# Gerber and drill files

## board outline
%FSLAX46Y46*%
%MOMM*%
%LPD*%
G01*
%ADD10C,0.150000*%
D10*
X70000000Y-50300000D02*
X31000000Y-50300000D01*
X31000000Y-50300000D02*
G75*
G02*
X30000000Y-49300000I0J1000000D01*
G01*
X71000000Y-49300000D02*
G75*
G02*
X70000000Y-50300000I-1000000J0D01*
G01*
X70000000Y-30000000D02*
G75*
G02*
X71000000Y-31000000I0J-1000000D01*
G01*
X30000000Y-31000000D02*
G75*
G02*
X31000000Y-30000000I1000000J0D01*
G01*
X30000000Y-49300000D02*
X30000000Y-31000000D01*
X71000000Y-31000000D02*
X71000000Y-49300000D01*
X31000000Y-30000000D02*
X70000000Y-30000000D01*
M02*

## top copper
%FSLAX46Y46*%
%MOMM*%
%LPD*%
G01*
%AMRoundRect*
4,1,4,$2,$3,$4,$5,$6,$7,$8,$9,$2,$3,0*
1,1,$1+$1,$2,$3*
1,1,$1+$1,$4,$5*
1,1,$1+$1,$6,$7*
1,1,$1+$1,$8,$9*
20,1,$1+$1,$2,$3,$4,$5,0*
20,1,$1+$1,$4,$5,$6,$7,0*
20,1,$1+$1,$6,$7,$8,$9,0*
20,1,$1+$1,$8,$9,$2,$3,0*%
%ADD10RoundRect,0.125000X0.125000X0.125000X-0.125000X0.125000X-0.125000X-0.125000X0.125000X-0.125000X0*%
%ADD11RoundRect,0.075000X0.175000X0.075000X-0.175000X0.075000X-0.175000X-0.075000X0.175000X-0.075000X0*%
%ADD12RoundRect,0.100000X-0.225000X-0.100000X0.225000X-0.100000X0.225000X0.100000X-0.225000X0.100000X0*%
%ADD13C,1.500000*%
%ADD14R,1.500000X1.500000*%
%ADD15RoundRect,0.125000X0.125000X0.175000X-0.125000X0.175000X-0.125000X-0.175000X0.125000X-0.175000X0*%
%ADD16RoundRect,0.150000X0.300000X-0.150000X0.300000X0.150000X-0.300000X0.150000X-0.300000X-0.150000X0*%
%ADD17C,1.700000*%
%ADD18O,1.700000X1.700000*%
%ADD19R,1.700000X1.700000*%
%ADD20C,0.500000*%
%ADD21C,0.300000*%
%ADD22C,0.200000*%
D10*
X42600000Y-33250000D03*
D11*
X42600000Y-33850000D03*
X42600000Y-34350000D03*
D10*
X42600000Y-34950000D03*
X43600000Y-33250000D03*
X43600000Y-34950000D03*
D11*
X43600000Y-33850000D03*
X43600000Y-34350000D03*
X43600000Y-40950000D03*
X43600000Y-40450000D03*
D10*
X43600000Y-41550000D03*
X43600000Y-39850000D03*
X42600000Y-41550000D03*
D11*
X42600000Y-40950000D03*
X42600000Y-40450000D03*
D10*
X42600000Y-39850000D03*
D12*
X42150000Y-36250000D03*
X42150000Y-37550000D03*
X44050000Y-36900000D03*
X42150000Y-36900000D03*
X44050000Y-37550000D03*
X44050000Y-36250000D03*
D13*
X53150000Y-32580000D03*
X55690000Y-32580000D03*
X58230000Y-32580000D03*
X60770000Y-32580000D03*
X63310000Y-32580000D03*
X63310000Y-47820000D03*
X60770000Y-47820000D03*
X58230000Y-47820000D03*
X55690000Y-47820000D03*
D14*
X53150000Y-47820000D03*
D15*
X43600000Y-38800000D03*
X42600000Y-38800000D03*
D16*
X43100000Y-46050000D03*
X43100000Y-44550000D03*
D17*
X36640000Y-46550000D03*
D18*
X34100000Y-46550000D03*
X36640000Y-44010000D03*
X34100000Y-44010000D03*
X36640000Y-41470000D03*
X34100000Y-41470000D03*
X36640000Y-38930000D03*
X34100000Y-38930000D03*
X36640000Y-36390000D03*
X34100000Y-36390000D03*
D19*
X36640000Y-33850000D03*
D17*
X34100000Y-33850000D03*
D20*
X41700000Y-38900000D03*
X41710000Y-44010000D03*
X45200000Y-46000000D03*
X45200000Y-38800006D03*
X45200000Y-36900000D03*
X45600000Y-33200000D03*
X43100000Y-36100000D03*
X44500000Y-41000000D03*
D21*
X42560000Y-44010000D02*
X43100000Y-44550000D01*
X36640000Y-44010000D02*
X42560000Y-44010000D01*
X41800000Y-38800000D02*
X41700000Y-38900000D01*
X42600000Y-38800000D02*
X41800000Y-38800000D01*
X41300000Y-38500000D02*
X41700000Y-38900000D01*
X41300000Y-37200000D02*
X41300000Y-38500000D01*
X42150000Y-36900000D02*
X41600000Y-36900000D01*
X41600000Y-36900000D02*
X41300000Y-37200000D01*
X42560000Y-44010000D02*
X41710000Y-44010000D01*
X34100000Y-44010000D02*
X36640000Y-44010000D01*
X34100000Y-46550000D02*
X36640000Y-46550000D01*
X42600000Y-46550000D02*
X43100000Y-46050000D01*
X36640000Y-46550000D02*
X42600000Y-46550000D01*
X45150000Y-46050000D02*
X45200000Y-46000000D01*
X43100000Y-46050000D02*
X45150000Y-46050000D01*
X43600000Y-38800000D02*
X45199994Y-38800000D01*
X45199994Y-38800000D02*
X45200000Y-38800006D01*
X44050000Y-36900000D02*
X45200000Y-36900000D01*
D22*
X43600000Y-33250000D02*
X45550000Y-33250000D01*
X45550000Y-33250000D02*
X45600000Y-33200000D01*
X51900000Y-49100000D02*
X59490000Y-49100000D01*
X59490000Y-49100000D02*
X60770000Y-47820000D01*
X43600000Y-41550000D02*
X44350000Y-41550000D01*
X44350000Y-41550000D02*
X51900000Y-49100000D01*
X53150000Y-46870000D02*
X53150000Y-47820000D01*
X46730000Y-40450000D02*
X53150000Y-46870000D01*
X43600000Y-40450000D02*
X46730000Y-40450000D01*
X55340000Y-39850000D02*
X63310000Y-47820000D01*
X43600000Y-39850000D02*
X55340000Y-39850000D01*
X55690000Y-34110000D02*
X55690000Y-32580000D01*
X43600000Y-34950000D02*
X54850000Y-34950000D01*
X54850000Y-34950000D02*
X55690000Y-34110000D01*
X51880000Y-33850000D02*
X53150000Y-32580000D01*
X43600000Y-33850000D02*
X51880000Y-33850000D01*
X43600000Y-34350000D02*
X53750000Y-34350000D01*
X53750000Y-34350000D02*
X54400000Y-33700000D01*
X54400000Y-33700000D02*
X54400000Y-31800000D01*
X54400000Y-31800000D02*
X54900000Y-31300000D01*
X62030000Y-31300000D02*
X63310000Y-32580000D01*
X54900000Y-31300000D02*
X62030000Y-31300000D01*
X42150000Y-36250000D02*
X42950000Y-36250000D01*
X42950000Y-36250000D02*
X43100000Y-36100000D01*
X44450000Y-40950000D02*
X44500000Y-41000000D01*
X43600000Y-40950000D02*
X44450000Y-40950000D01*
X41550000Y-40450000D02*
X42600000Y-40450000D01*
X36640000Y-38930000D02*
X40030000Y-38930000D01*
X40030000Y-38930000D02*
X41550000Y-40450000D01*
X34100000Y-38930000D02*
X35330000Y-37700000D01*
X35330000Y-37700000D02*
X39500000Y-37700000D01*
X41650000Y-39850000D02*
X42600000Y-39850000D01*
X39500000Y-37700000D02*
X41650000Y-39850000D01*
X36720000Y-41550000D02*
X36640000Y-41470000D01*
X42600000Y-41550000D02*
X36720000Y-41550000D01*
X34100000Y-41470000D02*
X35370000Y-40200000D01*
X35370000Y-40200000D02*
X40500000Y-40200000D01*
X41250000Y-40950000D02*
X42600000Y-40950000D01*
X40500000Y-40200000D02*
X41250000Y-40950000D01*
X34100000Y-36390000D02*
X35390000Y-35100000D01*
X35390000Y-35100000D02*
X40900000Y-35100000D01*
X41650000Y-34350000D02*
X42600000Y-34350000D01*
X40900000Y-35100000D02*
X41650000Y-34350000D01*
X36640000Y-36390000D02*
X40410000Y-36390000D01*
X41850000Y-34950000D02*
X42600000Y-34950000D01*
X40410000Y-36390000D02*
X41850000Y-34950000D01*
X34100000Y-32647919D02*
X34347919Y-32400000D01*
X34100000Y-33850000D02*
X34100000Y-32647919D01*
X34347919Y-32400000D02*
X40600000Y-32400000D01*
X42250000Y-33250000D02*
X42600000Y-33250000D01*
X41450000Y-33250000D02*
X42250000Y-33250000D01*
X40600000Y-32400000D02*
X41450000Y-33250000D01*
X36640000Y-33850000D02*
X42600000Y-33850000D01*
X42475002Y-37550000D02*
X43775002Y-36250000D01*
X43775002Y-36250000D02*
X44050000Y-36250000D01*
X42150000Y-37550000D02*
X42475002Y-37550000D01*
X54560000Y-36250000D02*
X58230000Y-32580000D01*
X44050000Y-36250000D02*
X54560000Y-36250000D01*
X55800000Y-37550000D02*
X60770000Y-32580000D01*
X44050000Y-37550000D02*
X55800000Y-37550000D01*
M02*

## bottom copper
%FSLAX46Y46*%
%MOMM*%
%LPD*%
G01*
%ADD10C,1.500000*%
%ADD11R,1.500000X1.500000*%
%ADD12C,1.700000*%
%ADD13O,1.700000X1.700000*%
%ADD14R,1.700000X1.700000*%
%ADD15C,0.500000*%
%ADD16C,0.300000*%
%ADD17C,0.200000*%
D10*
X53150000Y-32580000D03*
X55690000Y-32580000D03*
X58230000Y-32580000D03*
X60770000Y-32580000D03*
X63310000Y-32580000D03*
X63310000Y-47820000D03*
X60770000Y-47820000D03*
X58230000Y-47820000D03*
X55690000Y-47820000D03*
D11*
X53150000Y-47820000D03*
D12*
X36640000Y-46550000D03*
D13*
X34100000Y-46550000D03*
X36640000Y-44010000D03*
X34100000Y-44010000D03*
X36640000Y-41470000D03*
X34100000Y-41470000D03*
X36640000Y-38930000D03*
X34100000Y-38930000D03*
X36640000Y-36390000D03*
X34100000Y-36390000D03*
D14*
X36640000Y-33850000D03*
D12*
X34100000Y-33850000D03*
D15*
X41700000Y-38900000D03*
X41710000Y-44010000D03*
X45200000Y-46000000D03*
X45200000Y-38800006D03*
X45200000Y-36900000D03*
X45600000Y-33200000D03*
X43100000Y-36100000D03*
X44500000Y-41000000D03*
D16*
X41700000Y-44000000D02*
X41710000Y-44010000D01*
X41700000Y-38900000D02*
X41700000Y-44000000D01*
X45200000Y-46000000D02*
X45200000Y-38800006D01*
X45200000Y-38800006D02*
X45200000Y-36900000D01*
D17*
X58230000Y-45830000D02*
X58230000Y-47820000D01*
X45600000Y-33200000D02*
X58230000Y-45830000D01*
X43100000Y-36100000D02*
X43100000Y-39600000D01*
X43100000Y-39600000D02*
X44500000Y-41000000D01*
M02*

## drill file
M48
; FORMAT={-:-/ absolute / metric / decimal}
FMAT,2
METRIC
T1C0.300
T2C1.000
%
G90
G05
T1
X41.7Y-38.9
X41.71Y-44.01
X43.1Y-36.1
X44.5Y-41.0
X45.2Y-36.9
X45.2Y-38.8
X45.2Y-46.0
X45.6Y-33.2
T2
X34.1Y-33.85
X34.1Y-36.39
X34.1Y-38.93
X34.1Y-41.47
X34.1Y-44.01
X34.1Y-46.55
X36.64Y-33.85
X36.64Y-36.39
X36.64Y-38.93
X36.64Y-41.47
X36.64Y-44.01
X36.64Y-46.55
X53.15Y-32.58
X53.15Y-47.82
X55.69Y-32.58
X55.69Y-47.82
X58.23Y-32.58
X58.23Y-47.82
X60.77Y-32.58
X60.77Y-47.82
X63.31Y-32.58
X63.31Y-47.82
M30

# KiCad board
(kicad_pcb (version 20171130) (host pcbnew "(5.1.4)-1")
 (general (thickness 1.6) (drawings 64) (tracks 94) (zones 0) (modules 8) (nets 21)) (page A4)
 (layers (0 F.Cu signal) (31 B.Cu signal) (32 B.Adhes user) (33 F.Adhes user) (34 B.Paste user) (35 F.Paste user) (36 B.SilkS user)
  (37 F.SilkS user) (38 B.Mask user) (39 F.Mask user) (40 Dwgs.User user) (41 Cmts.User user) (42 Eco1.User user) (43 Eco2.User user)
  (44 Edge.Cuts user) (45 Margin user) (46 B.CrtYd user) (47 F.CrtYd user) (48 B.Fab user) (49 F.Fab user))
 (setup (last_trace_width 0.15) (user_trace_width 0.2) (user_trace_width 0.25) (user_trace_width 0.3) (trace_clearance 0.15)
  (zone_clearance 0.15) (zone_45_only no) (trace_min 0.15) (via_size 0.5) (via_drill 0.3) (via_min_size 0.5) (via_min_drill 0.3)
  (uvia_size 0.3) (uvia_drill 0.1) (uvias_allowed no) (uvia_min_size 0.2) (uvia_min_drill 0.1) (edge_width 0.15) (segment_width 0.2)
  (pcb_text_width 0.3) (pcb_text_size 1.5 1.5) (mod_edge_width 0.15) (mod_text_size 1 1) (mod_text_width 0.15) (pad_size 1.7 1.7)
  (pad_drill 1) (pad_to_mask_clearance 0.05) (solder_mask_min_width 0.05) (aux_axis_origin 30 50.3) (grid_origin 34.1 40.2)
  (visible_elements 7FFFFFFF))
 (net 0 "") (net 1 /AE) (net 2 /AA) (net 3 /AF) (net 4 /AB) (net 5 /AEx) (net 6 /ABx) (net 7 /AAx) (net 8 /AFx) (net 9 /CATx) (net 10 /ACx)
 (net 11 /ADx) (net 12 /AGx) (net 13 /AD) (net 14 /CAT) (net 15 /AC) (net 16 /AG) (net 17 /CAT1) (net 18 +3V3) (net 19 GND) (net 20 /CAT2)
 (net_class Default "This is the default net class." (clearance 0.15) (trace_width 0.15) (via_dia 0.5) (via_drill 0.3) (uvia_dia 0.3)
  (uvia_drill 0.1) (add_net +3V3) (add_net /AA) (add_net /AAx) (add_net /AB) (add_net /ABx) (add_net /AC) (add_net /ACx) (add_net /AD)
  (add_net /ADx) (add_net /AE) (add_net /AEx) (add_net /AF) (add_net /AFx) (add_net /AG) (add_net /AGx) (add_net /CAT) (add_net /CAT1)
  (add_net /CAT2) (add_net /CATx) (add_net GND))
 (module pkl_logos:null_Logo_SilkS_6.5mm (layer B.Cu) (at 52.7 40.2 90)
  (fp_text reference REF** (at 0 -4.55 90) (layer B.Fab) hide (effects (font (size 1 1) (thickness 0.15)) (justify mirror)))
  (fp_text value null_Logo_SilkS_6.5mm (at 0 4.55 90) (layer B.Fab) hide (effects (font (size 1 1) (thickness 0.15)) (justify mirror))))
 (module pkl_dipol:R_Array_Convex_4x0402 (layer F.Cu) (at 43.1 34.1 180) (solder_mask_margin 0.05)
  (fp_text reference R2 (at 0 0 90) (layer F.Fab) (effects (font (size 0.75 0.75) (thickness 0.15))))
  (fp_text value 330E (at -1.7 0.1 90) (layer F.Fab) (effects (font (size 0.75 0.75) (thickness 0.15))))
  (pad 8 smd roundrect (at 0.5 0.85 180) (size 0.5 0.5) (layers F.Cu F.Paste F.Mask) (roundrect_rratio 0.25) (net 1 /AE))
  (pad 6 smd roundrect (at 0.5 0.25 180) (size 0.5 0.3) (layers F.Cu F.Paste F.Mask) (roundrect_rratio 0.25) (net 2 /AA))
  (pad 4 smd roundrect (at 0.5 -0.25 180) (size 0.5 0.3) (layers F.Cu F.Paste F.Mask) (roundrect_rratio 0.25) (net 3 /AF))
  (pad 2 smd roundrect (at 0.5 -0.85 180) (size 0.5 0.5) (layers F.Cu F.Paste F.Mask) (roundrect_rratio 0.25) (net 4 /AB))
  (pad 7 smd roundrect (at -0.5 0.85 180) (size 0.5 0.5) (layers F.Cu F.Paste F.Mask) (roundrect_rratio 0.25) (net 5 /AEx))
  (pad 1 smd roundrect (at -0.5 -0.85 180) (size 0.5 0.5) (layers F.Cu F.Paste F.Mask) (roundrect_rratio 0.25) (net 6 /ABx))
  (pad 5 smd roundrect (at -0.5 0.25 180) (size 0.5 0.3) (layers F.Cu F.Paste F.Mask) (roundrect_rratio 0.25) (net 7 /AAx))
  (pad 3 smd roundrect (at -0.5 -0.25 180) (size 0.5 0.3) (layers F.Cu F.Paste F.Mask) (roundrect_rratio 0.25) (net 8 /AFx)))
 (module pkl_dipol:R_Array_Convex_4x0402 (layer F.Cu) (at 43.1 40.7 180) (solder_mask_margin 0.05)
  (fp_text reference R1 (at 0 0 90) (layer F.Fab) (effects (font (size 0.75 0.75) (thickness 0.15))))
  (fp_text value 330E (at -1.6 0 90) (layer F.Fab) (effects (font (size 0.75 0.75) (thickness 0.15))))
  (pad 3 smd roundrect (at -0.5 -0.25 180) (size 0.5 0.3) (layers F.Cu F.Paste F.Mask) (roundrect_rratio 0.25) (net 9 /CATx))
  (pad 5 smd roundrect (at -0.5 0.25 180) (size 0.5 0.3) (layers F.Cu F.Paste F.Mask) (roundrect_rratio 0.25) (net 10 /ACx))
  (pad 1 smd roundrect (at -0.5 -0.85 180) (size 0.5 0.5) (layers F.Cu F.Paste F.Mask) (roundrect_rratio 0.25) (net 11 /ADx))
  (pad 7 smd roundrect (at -0.5 0.85 180) (size 0.5 0.5) (layers F.Cu F.Paste F.Mask) (roundrect_rratio 0.25) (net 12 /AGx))
  (pad 2 smd roundrect (at 0.5 -0.85 180) (size 0.5 0.5) (layers F.Cu F.Paste F.Mask) (roundrect_rratio 0.25) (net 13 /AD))
  (pad 4 smd roundrect (at 0.5 -0.25 180) (size 0.5 0.3) (layers F.Cu F.Paste F.Mask) (roundrect_rratio 0.25) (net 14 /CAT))
  (pad 6 smd roundrect (at 0.5 0.25 180) (size 0.5 0.3) (layers F.Cu F.Paste F.Mask) (roundrect_rratio 0.25) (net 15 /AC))
  (pad 8 smd roundrect (at 0.5 0.85 180) (size 0.5 0.5) (layers F.Cu F.Paste F.Mask) (roundrect_rratio 0.25) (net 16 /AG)))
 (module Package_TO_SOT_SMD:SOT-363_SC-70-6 (layer F.Cu) (at 43.1 36.9)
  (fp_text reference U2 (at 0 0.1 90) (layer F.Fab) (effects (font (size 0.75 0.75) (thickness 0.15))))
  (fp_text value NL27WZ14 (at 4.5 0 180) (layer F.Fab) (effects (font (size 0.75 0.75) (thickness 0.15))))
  (pad 1 smd roundrect (at -0.95 -0.65) (size 0.65 0.4) (layers F.Cu F.Paste F.Mask) (roundrect_rratio 0.25) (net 9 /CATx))
  (pad 3 smd roundrect (at -0.95 0.65) (size 0.65 0.4) (layers F.Cu F.Paste F.Mask) (roundrect_rratio 0.25) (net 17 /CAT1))
  (pad 5 smd roundrect (at 0.95 0) (size 0.65 0.4) (layers F.Cu F.Paste F.Mask) (roundrect_rratio 0.25) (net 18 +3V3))
  (pad 2 smd roundrect (at -0.95 0) (size 0.65 0.4) (layers F.Cu F.Paste F.Mask) (roundrect_rratio 0.25) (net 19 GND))
  (pad 4 smd roundrect (at 0.95 0.65) (size 0.65 0.4) (layers F.Cu F.Paste F.Mask) (roundrect_rratio 0.25) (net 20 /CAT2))
  (pad 6 smd roundrect (at 0.95 -0.65) (size 0.65 0.4) (layers F.Cu F.Paste F.Mask) (roundrect_rratio 0.25) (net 17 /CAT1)))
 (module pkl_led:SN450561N (layer F.Cu) (at 53.15 47.82 90)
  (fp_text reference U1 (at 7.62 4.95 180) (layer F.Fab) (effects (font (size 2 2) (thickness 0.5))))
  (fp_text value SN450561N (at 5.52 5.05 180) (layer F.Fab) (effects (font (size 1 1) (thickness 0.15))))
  (pad 10 thru_hole circle (at 15.24 0 90) (size 1.5 1.5) (drill 1) (layers *.Cu *.Mask) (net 7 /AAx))
  (pad 9 thru_hole circle (at 15.24 2.54 90) (size 1.5 1.5) (drill 1) (layers *.Cu *.Mask) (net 6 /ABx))
  (pad 8 thru_hole circle (at 15.24 5.08 90) (size 1.5 1.5) (drill 1) (layers *.Cu *.Mask) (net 17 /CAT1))
  (pad 7 thru_hole circle (at 15.24 7.62 90) (size 1.5 1.5) (drill 1) (layers *.Cu *.Mask) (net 20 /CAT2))
  (pad 6 thru_hole circle (at 15.24 10.16 90) (size 1.5 1.5) (drill 1) (layers *.Cu *.Mask) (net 8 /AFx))
  (pad 5 thru_hole circle (at 0 10.16 90) (size 1.5 1.5) (drill 1) (layers *.Cu *.Mask) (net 12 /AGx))
  (pad 4 thru_hole circle (at 0 7.62 90) (size 1.5 1.5) (drill 1) (layers *.Cu *.Mask) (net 11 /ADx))
  (pad 3 thru_hole circle (at 0 5.08 90) (size 1.5 1.5) (drill 1) (layers *.Cu *.Mask) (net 5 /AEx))
  (pad 2 thru_hole circle (at 0 2.54 90) (size 1.5 1.5) (drill 1) (layers *.Cu *.Mask))
  (pad 1 thru_hole rect (at 0 0 90) (size 1.5 1.5) (drill 1) (layers *.Cu *.Mask) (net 10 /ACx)))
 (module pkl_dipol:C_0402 (layer F.Cu) (at 43.1 38.8 180)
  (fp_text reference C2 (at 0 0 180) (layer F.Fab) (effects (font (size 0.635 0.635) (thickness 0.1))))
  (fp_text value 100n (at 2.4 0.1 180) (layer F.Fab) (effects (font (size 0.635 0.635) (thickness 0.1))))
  (pad 1 smd roundrect (at -0.5 0 180) (size 0.5 0.6) (layers F.Cu F.Paste F.Mask) (roundrect_rratio 0.25) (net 18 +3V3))
  (pad 2 smd roundrect (at 0.5 0 180) (size 0.5 0.6) (layers F.Cu F.Paste F.Mask) (roundrect_rratio 0.25) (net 19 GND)))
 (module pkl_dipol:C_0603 (layer F.Cu) (at 43.1 45.3 90)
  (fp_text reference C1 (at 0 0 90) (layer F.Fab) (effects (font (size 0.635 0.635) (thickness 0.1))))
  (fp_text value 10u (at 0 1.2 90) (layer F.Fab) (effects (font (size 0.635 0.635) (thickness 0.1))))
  (pad 1 smd roundrect (at -0.75 0 90) (size 0.6 0.9) (layers F.Cu F.Paste F.Mask) (roundrect_rratio 0.25) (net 18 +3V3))
  (pad 2 smd roundrect (at 0.75 0 90) (size 0.6 0.9) (layers F.Cu F.Paste F.Mask) (roundrect_rratio 0.25) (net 19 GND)))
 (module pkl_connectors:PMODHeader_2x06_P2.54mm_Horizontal (layer F.Cu) (at 36.64 46.55 180)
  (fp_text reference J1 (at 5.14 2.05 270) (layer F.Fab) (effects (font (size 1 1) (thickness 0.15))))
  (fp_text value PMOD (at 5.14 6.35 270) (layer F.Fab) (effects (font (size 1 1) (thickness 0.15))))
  (pad 6 thru_hole circle (at 0 0 180) (size 1.7 1.7) (drill 1) (layers *.Cu *.Mask) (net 18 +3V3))
  (pad 12 thru_hole oval (at 2.54 0 180) (size 1.7 1.7) (drill 1) (layers *.Cu *.Mask) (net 18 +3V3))
  (pad 5 thru_hole oval (at 0 2.54 180) (size 1.7 1.7) (drill 1) (layers *.Cu *.Mask) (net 19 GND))
  (pad 11 thru_hole oval (at 2.54 2.54 180) (size 1.7 1.7) (drill 1) (layers *.Cu *.Mask) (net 19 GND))
  (pad 4 thru_hole oval (at 0 5.08 180) (size 1.7 1.7) (drill 1) (layers *.Cu *.Mask) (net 13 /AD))
  (pad 10 thru_hole oval (at 2.54 5.08 180) (size 1.7 1.7) (drill 1) (layers *.Cu *.Mask) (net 14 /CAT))
  (pad 3 thru_hole oval (at 0 7.62 180) (size 1.7 1.7) (drill 1) (layers *.Cu *.Mask) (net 15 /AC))
  (pad 9 thru_hole oval (at 2.54 7.62 180) (size 1.7 1.7) (drill 1) (layers *.Cu *.Mask) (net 16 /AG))
  (pad 2 thru_hole oval (at 0 10.16 180) (size 1.7 1.7) (drill 1) (layers *.Cu *.Mask) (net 4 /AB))
  (pad 8 thru_hole oval (at 2.54 10.16 180) (size 1.7 1.7) (drill 1) (layers *.Cu *.Mask) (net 3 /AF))
  (pad 1 thru_hole rect (at 0 12.7 180) (size 1.7 1.7) (drill 1) (layers *.Cu *.Mask) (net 2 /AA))
  (pad 7 thru_hole circle (at 2.54 12.7 180) (size 1.7 1.7) (drill 1) (layers *.Cu *.Mask) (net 1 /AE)))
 (gr_line (start 70 50.3) (end 31 50.3) (layer Edge.Cuts) (width 0.15))
 (gr_arc (start 31 49.3) (end 30 49.3) (angle -90) (layer Edge.Cuts) (width 0.15))
 (gr_arc (start 70 49.3) (end 70 50.3) (angle -90) (layer Edge.Cuts) (width 0.15))
 (gr_arc (start 70 31) (end 71 31) (angle -90) (layer Edge.Cuts) (width 0.15))
 (gr_arc (start 31 31) (end 31 30) (angle -90) (layer Edge.Cuts) (width 0.15))
 (gr_line (start 30 49.3) (end 30 31) (layer Edge.Cuts) (width 0.15))
 (gr_line (start 71 31) (end 71 49.3) (layer Edge.Cuts) (width 0.15))
 (gr_line (start 31 30) (end 70 30) (layer Edge.Cuts) (width 0.15))
 (segment (start 42.56 44.01) (end 43.1 44.55) (width 0.3) (layer F.Cu) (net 19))
 (segment (start 36.64 44.01) (end 42.56 44.01) (width 0.3) (layer F.Cu) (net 19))
 (via (at 41.7 38.9) (size 0.5) (drill 0.3) (layers F.Cu B.Cu) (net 19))
 (segment (start 41.8 38.8) (end 41.7 38.9) (width 0.3) (layer F.Cu) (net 19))
 (segment (start 42.6 38.8) (end 41.8 38.8) (width 0.3) (layer F.Cu) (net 19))
 (segment (start 41.3 38.5) (end 41.7 38.9) (width 0.3) (layer F.Cu) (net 19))
 (segment (start 41.3 37.2) (end 41.3 38.5) (width 0.3) (layer F.Cu) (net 19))
 (segment (start 42.15 36.9) (end 41.6 36.9) (width 0.3) (layer F.Cu) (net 19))
 (segment (start 41.6 36.9) (end 41.3 37.2) (width 0.3) (layer F.Cu) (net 19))
 (segment (start 42.56 44.01) (end 41.71 44.01) (width 0.3) (layer F.Cu) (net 19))
 (segment (start 41.7 44) (end 41.71 44.01) (width 0.3) (layer B.Cu) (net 19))
 (via (at 41.71 44.01) (size 0.5) (drill 0.3) (layers F.Cu B.Cu) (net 19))
 (segment (start 41.7 38.9) (end 41.7 44) (width 0.3) (layer B.Cu) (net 19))
 (segment (start 34.1 44.01) (end 36.64 44.01) (width 0.3) (layer F.Cu) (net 19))
 (segment (start 34.1 46.55) (end 36.64 46.55) (width 0.3) (layer F.Cu) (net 18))
 (segment (start 42.6 46.55) (end 43.1 46.05) (width 0.3) (layer F.Cu) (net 18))
 (segment (start 36.64 46.55) (end 42.6 46.55) (width 0.3) (layer F.Cu) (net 18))
 (segment (start 45.15 46.05) (end 45.2 46) (width 0.3) (layer F.Cu) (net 18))
 (via (at 45.2 46) (size 0.5) (drill 0.3) (layers F.Cu B.Cu) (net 18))
 (segment (start 43.1 46.05) (end 45.15 46.05) (width 0.3) (layer F.Cu) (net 18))
 (via (at 45.2 38.800006) (size 0.5) (drill 0.3) (layers F.Cu B.Cu) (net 18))
 (segment (start 43.6 38.8) (end 45.199994 38.8) (width 0.3) (layer F.Cu) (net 18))
 (segment (start 45.199994 38.8) (end 45.2 38.800006) (width 0.3) (layer F.Cu) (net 18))
 (segment (start 45.2 46) (end 45.2 38.800006) (width 0.3) (layer B.Cu) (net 18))
 (via (at 45.2 36.9) (size 0.5) (drill 0.3) (layers F.Cu B.Cu) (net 18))
 (segment (start 45.2 38.800006) (end 45.2 36.9) (width 0.3) (layer B.Cu) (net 18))
 (segment (start 44.05 36.9) (end 45.2 36.9) (width 0.3) (layer F.Cu) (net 18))
 (via (at 45.6 33.2) (size 0.5) (drill 0.3) (layers F.Cu B.Cu) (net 5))
 (segment (start 43.6 33.25) (end 45.55 33.25) (width 0.2) (layer F.Cu) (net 5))
 (segment (start 45.55 33.25) (end 45.6 33.2) (width 0.2) (layer F.Cu) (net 5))
 (segment (start 58.23 45.83) (end 58.23 47.82) (width 0.2) (layer B.Cu) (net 5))
 (segment (start 45.6 33.2) (end 58.23 45.83) (width 0.2) (layer B.Cu) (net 5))
 (segment (start 51.9 49.1) (end 59.49 49.1) (width 0.2) (layer F.Cu) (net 11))
 (segment (start 59.49 49.1) (end 60.77 47.82) (width 0.2) (layer F.Cu) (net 11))
 (segment (start 43.6 41.55) (end 44.35 41.55) (width 0.2) (layer F.Cu) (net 11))
 (segment (start 44.35 41.55) (end 51.9 49.1) (width 0.2) (layer F.Cu) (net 11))
 (segment (start 53.15 46.87) (end 53.15 47.82) (width 0.2) (layer F.Cu) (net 10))
 (segment (start 46.73 40.45) (end 53.15 46.87) (width 0.2) (layer F.Cu) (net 10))
 (segment (start 43.6 40.45) (end 46.73 40.45) (width 0.2) (layer F.Cu) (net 10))
 (segment (start 55.34 39.85) (end 63.31 47.82) (width 0.2) (layer F.Cu) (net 12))
 (segment (start 43.6 39.85) (end 55.34 39.85) (width 0.2) (layer F.Cu) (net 12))
 (segment (start 55.69 34.11) (end 55.69 32.58) (width 0.2) (layer F.Cu) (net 6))
 (segment (start 43.6 34.95) (end 54.85 34.95) (width 0.2) (layer F.Cu) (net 6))
 (segment (start 54.85 34.95) (end 55.69 34.11) (width 0.2) (layer F.Cu) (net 6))
 (segment (start 51.88 33.85) (end 53.15 32.58) (width 0.2) (layer F.Cu) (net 7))
 (segment (start 43.6 33.85) (end 51.88 33.85) (width 0.2) (layer F.Cu) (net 7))
 (segment (start 43.6 34.35) (end 53.75 34.35) (width 0.2) (layer F.Cu) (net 8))
 (segment (start 53.75 34.35) (end 54.4 33.7) (width 0.2) (layer F.Cu) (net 8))
 (segment (start 54.4 33.7) (end 54.4 31.8) (width 0.2) (layer F.Cu) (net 8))
 (segment (start 54.4 31.8) (end 54.9 31.3) (width 0.2) (layer F.Cu) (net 8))
 (segment (start 62.03 31.3) (end 63.31 32.58) (width 0.2) (layer F.Cu) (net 8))
 (segment (start 54.9 31.3) (end 62.03 31.3) (width 0.2) (layer F.Cu) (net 8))
 (via (at 43.1 36.1) (size 0.5) (drill 0.3) (layers F.Cu B.Cu) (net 9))
 (segment (start 42.15 36.25) (end 42.95 36.25) (width 0.2) (layer F.Cu) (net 9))
 (segment (start 42.95 36.25) (end 43.1 36.1) (width 0.2) (layer F.Cu) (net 9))
 (via (at 44.5 41) (size 0.5) (drill 0.3) (layers F.Cu B.Cu) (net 9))
 (segment (start 43.1 36.1) (end 43.1 39.6) (width 0.2) (layer B.Cu) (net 9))
 (segment (start 43.1 39.6) (end 44.5 41) (width 0.2) (layer B.Cu) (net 9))
 (segment (start 44.45 40.95) (end 44.5 41) (width 0.2) (layer F.Cu) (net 9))
 (segment (start 43.6 40.95) (end 44.45 40.95) (width 0.2) (layer F.Cu) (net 9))
 (segment (start 41.55 40.45) (end 42.6 40.45) (width 0.2) (layer F.Cu) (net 15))
 (segment (start 36.64 38.93) (end 40.03 38.93) (width 0.2) (layer F.Cu) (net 15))
 (segment (start 40.03 38.93) (end 41.55 40.45) (width 0.2) (layer F.Cu) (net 15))
 (segment (start 34.1 38.93) (end 35.33 37.7) (width 0.2) (layer F.Cu) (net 16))
 (segment (start 35.33 37.7) (end 39.5 37.7) (width 0.2) (layer F.Cu) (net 16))
 (segment (start 41.65 39.85) (end 42.6 39.85) (width 0.2) (layer F.Cu) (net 16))
 (segment (start 39.5 37.7) (end 41.65 39.85) (width 0.2) (layer F.Cu) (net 16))
 (segment (start 36.72 41.55) (end 36.64 41.47) (width 0.2) (layer F.Cu) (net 13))
 (segment (start 42.6 41.55) (end 36.72 41.55) (width 0.2) (layer F.Cu) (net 13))
 (segment (start 34.1 41.47) (end 35.37 40.2) (width 0.2) (layer F.Cu) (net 14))
 (segment (start 35.37 40.2) (end 40.5 40.2) (width 0.2) (layer F.Cu) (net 14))
 (segment (start 41.25 40.95) (end 42.6 40.95) (width 0.2) (layer F.Cu) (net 14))
 (segment (start 40.5 40.2) (end 41.25 40.95) (width 0.2) (layer F.Cu) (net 14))
 (segment (start 34.1 36.39) (end 35.39 35.1) (width 0.2) (layer F.Cu) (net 3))
 (segment (start 35.39 35.1) (end 40.9 35.1) (width 0.2) (layer F.Cu) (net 3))
 (segment (start 41.65 34.35) (end 42.6 34.35) (width 0.2) (layer F.Cu) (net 3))
 (segment (start 40.9 35.1) (end 41.65 34.35) (width 0.2) (layer F.Cu) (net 3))
 (segment (start 36.64 36.39) (end 40.41 36.39) (width 0.2) (layer F.Cu) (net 4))
 (segment (start 41.85 34.95) (end 42.6 34.95) (width 0.2) (layer F.Cu) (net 4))
 (segment (start 40.41 36.39) (end 41.85 34.95) (width 0.2) (layer F.Cu) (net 4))
 (segment (start 34.1 32.647919) (end 34.347919 32.4) (width 0.2) (layer F.Cu) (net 1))
 (segment (start 34.1 33.85) (end 34.1 32.647919) (width 0.2) (layer F.Cu) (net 1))
 (segment (start 34.347919 32.4) (end 40.6 32.4) (width 0.2) (layer F.Cu) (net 1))
 (segment (start 42.25 33.25) (end 42.6 33.25) (width 0.2) (layer F.Cu) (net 1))
 (segment (start 41.45 33.25) (end 42.25 33.25) (width 0.2) (layer F.Cu) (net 1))
 (segment (start 40.6 32.4) (end 41.45 33.25) (width 0.2) (layer F.Cu) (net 1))
 (segment (start 36.64 33.85) (end 42.6 33.85) (width 0.2) (layer F.Cu) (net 2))
 (segment (start 42.475002 37.55) (end 43.775002 36.25) (width 0.2) (layer F.Cu) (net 17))
 (segment (start 43.775002 36.25) (end 44.05 36.25) (width 0.2) (layer F.Cu) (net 17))
 (segment (start 42.15 37.55) (end 42.475002 37.55) (width 0.2) (layer F.Cu) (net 17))
 (segment (start 54.56 36.25) (end 58.23 32.58) (width 0.2) (layer F.Cu) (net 17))
 (segment (start 44.05 36.25) (end 54.56 36.25) (width 0.2) (layer F.Cu) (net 17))
 (segment (start 55.8 37.55) (end 60.77 32.58) (width 0.2) (layer F.Cu) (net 20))
 (segment (start 44.05 37.55) (end 55.8 37.55) (width 0.2) (layer F.Cu) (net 20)))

